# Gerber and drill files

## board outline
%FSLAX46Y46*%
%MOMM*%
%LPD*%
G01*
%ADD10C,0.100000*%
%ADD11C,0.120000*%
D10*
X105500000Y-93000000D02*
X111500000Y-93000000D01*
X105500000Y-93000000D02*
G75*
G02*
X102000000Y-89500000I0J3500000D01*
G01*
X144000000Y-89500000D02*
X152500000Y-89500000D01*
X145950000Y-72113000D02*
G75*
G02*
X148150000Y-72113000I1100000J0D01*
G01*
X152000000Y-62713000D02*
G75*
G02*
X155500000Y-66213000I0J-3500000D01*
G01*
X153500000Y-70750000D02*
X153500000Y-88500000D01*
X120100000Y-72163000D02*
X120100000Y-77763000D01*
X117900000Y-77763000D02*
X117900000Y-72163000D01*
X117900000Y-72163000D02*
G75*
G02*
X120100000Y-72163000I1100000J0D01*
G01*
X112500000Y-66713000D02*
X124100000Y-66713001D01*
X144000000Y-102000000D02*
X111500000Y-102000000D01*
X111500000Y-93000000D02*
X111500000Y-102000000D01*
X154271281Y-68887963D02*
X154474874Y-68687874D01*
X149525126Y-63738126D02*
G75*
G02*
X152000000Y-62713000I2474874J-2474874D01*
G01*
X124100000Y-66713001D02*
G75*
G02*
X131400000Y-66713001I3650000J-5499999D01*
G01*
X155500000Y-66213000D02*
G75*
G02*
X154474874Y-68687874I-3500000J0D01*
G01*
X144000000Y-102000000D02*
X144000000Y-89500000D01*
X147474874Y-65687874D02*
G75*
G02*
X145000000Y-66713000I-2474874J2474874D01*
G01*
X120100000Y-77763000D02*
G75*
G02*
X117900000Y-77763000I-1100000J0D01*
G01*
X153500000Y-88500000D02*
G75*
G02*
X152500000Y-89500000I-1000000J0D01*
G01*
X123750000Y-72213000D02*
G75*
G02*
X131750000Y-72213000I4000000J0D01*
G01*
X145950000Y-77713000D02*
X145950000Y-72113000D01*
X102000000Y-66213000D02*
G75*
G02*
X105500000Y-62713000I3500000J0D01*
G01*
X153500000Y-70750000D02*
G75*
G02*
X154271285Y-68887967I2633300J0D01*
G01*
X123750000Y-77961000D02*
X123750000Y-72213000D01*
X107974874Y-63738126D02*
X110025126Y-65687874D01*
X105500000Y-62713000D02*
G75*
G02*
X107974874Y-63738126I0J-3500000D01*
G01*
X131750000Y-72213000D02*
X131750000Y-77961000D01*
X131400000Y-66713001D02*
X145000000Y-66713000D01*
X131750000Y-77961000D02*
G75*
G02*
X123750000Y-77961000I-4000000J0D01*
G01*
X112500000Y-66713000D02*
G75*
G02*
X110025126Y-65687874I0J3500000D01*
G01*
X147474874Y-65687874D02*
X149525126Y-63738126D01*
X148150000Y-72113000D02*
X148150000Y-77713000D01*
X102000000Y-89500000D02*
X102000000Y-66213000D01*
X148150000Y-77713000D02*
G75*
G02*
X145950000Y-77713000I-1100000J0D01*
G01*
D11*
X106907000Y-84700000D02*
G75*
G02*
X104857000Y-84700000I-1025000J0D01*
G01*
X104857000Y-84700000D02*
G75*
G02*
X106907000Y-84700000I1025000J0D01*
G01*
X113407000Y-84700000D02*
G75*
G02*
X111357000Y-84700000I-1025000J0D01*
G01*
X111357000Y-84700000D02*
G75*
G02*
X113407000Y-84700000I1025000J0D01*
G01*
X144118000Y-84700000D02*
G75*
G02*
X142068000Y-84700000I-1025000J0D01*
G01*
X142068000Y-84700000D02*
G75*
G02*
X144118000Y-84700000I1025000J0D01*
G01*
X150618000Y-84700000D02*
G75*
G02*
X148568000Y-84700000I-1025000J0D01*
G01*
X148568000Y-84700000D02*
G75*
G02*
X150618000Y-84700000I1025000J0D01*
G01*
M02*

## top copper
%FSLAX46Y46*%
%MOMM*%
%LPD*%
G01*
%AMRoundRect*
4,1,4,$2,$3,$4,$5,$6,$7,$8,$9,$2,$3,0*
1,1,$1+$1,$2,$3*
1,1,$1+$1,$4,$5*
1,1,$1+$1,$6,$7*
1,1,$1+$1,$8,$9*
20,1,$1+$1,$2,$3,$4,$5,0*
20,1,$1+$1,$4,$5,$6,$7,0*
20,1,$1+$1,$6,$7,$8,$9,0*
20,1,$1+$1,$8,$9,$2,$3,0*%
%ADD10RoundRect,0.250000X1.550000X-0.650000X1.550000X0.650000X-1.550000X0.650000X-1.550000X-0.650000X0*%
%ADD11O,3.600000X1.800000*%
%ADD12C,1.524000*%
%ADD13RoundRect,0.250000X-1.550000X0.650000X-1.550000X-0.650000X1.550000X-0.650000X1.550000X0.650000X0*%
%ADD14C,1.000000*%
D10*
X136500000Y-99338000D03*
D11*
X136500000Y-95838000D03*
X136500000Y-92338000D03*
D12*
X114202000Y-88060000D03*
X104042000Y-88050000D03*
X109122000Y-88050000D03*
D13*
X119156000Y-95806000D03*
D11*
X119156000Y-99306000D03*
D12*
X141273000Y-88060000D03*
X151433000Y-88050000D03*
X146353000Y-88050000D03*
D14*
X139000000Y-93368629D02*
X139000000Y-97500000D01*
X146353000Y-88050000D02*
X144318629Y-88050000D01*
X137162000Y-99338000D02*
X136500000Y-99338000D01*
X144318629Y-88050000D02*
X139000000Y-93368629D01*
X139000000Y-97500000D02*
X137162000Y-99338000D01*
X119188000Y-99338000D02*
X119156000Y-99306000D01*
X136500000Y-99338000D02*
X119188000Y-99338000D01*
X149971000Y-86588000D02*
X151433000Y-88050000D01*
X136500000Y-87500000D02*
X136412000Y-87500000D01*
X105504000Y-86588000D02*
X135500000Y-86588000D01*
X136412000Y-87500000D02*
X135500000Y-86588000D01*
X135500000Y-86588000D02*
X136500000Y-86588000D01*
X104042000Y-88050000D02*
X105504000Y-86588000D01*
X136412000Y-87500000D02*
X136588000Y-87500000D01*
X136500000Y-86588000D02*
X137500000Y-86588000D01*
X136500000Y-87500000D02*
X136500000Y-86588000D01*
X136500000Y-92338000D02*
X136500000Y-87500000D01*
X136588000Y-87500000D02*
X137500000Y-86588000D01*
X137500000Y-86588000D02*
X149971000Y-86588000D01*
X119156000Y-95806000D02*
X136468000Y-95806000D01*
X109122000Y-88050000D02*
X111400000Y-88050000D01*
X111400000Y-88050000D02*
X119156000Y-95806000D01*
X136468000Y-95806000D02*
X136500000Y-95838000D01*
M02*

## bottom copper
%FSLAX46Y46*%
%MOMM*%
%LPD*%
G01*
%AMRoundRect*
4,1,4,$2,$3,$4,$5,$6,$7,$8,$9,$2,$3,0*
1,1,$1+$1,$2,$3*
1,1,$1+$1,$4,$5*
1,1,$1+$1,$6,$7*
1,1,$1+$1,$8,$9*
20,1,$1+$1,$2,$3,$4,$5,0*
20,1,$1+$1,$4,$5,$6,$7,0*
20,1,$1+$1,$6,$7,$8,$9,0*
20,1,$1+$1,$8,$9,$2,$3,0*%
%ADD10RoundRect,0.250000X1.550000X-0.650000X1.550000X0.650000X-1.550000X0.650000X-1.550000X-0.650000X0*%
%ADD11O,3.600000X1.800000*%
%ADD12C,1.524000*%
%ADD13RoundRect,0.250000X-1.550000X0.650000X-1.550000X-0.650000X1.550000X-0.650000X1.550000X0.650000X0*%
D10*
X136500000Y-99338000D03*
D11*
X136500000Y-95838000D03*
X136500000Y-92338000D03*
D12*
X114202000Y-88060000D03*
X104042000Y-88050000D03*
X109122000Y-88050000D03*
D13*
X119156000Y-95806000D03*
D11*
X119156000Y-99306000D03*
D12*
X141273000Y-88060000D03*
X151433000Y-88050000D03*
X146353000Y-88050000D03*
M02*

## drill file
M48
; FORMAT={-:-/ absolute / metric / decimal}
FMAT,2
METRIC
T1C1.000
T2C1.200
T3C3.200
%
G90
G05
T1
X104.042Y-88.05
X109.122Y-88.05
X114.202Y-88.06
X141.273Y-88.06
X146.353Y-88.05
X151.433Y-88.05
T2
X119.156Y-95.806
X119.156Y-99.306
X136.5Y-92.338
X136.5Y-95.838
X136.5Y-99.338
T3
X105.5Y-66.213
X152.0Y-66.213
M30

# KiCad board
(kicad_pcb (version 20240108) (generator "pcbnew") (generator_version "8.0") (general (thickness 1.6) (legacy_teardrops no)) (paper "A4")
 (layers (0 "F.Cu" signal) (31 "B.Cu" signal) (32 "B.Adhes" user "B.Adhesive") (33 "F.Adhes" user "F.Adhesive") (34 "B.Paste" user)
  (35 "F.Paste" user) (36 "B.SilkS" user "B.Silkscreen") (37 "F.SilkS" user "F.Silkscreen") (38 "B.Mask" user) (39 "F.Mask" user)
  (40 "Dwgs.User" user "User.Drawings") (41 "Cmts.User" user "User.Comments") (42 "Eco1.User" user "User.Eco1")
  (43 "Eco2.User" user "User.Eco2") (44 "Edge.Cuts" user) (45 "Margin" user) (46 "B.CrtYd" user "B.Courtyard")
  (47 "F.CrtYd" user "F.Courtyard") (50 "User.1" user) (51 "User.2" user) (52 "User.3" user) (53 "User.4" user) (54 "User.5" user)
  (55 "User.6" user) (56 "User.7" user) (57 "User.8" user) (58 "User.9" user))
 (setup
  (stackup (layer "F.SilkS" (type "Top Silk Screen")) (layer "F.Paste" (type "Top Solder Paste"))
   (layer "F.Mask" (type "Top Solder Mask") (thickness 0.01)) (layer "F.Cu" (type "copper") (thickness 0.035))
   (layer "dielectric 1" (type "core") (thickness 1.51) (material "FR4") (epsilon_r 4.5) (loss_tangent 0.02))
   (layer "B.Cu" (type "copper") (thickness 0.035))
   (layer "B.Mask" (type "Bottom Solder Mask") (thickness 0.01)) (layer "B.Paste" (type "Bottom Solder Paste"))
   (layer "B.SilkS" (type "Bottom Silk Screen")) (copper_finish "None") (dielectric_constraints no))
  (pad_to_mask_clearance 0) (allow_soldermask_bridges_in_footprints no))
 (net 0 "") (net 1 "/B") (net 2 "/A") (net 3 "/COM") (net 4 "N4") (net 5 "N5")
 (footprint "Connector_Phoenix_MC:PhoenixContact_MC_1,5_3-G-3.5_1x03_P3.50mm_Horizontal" (layer "F.Cu") (at 136.5 99.338 90)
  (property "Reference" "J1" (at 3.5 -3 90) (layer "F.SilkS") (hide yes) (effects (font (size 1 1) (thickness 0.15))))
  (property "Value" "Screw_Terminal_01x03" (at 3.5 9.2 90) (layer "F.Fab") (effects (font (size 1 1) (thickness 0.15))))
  (pad "1" thru_hole roundrect (at 0 0 90) (size 1.8 3.6) (drill 1.2) (layers "*.Cu" "*.Mask") (remove_unused_layers no)
   (roundrect_rratio 0.1388888889) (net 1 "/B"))
  (pad "2" thru_hole oval (at 3.5 0 90) (size 1.8 3.6) (drill 1.2) (layers "*.Cu" "*.Mask") (remove_unused_layers no) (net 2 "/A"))
  (pad "3" thru_hole oval (at 7 0 90) (size 1.8 3.6) (drill 1.2) (layers "*.Cu" "*.Mask") (remove_unused_layers no) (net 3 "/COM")))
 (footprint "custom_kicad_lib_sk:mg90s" (layer "F.Cu") (at 127.674 72.5)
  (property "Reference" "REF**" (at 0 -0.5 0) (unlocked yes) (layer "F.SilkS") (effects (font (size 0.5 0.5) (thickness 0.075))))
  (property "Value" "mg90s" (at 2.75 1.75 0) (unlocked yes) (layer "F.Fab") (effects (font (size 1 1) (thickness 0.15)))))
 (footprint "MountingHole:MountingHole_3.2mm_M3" (layer "F.Cu") (at 152 66.213)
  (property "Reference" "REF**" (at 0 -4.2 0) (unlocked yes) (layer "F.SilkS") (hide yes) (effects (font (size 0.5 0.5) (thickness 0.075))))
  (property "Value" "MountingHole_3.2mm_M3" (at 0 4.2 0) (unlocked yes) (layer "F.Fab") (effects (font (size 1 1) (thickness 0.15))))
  (pad "" np_thru_hole circle (at 0 0) (size 3.2 3.2) (drill 3.2) (layers "*.Cu" "*.Mask")))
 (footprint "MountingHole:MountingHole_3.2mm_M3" (layer "F.Cu") (at 105.5 66.213)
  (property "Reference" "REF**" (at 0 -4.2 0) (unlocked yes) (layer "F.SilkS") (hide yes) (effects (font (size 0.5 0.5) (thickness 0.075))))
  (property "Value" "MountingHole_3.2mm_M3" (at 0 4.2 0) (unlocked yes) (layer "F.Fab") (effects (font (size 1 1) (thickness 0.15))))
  (pad "" np_thru_hole circle (at 0 0) (size 3.2 3.2) (drill 3.2) (layers "F&B.Cu" "*.Mask")))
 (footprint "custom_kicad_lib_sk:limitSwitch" (layer "F.Cu") (at 109.122 87.5)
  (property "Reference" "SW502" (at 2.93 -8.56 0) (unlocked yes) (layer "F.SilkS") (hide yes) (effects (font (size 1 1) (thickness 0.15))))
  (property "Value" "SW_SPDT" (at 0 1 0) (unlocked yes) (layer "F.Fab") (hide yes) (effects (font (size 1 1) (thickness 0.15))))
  (fp_circle (center -3.24 -2.8) (end -2.215 -2.8) (stroke (width 0.12) (type default)) (fill none) (layer "Edge.Cuts"))
  (fp_circle (center 3.26 -2.8) (end 4.285 -2.8) (stroke (width 0.12) (type default)) (fill none) (layer "Edge.Cuts"))
  (pad "1" thru_hole circle (at 5.08 0.56) (size 1.524 1.524) (drill 1) (layers "*.Cu" "*.Mask") (remove_unused_layers no) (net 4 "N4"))
  (pad "2" thru_hole circle (at -5.08 0.55) (size 1.524 1.524) (drill 1) (layers "*.Cu" "*.Mask") (remove_unused_layers no) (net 3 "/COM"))
  (pad "3" thru_hole circle (at 0 0.55) (size 1.524 1.524) (drill 1) (layers "*.Cu" "*.Mask") (remove_unused_layers no) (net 2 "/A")))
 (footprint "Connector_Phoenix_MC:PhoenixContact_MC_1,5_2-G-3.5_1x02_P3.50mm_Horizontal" (layer "F.Cu") (at 119.156 95.806 -90)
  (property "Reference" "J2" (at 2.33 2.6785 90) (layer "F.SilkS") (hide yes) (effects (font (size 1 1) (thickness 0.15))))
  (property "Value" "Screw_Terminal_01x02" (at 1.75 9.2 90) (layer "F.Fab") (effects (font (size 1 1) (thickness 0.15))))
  (pad "1" thru_hole roundrect (at 0 0 270) (size 1.8 3.6) (drill 1.2) (layers "*.Cu" "*.Mask") (remove_unused_layers no)
   (roundrect_rratio 0.1388888889) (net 2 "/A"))
  (pad "2" thru_hole oval (at 3.5 0 270) (size 1.8 3.6) (drill 1.2) (layers "*.Cu" "*.Mask") (remove_unused_layers no) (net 1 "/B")))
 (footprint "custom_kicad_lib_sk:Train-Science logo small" (layer "F.Cu") (at 125.5 87.5)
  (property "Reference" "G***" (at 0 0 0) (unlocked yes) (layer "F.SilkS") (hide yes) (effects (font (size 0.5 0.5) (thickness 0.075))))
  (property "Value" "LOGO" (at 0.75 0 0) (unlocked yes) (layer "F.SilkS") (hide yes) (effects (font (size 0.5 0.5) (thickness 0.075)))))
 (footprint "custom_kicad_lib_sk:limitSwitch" (layer "B.Cu") (at 146.353 87.5 180)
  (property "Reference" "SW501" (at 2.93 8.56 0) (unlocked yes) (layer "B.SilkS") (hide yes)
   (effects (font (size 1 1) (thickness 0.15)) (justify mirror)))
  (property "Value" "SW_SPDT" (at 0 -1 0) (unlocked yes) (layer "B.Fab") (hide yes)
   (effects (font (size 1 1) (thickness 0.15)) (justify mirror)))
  (fp_circle (center 3.26 2.8) (end 4.285 2.8) (stroke (width 0.12) (type default)) (fill none) (layer "Edge.Cuts"))
  (fp_circle (center -3.24 2.8) (end -2.215 2.8) (stroke (width 0.12) (type default)) (fill none) (layer "Edge.Cuts"))
  (pad "1" thru_hole circle (at 5.08 -0.56 180) (size 1.524 1.524) (drill 1) (layers "*.Cu" "*.Mask") (remove_unused_layers no) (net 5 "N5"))
  (pad "2" thru_hole circle (at -5.08 -0.55 180) (size 1.524 1.524) (drill 1) (layers "*.Cu" "*.Mask") (remove_unused_layers no)
   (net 3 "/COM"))
  (pad "3" thru_hole circle (at 0 -0.55 180) (size 1.524 1.524) (drill 1) (layers "*.Cu" "*.Mask") (remove_unused_layers no) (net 1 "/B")))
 (gr_line (start 105.5 93) (end 111.5 93) (stroke (width 0.1) (type default)) (layer "Edge.Cuts"))
 (gr_arc (start 105.5 93) (mid 103.025126 91.974874) (end 102 89.5) (stroke (width 0.1) (type default)) (layer "Edge.Cuts"))
 (gr_line (start 144 89.5) (end 152.5 89.5) (stroke (width 0.1) (type default)) (layer "Edge.Cuts"))
 (gr_arc (start 145.95 72.113) (mid 147.05 71.013) (end 148.15 72.113) (stroke (width 0.1) (type default)) (layer "Edge.Cuts"))
 (gr_arc (start 152 62.713) (mid 154.474874 63.738126) (end 155.5 66.213) (stroke (width 0.1) (type default)) (layer "Edge.Cuts"))
 (gr_line (start 153.5 70.75) (end 153.5 88.5) (stroke (width 0.1) (type default)) (layer "Edge.Cuts"))
 (gr_line (start 120.1 72.163) (end 120.1 77.763) (stroke (width 0.1) (type default)) (layer "Edge.Cuts"))
 (gr_line (start 117.9 77.763) (end 117.9 72.163) (stroke (width 0.1) (type default)) (layer "Edge.Cuts"))
 (gr_arc (start 117.9 72.163) (mid 119 71.063) (end 120.1 72.163) (stroke (width 0.1) (type default)) (layer "Edge.Cuts"))
 (gr_line (start 112.5 66.713) (end 124.1 66.713001) (stroke (width 0.1) (type default)) (layer "Edge.Cuts"))
 (gr_line (start 144 102) (end 111.5 102) (stroke (width 0.1) (type default)) (layer "Edge.Cuts"))
 (gr_line (start 111.5 93) (end 111.5 102) (stroke (width 0.1) (type default)) (layer "Edge.Cuts"))
 (gr_line (start 154.271281 68.887963) (end 154.474874 68.687874) (stroke (width 0.1) (type default)) (layer "Edge.Cuts"))
 (gr_arc (start 149.525126 63.738126) (mid 150.660608 62.979421) (end 152 62.713) (stroke (width 0.1) (type default)) (layer "Edge.Cuts"))
 (gr_arc (start 124.1 66.713001) (mid 127.75 65.612054) (end 131.4 66.713001) (stroke (width 0.1) (type default)) (layer "Edge.Cuts"))
 (gr_arc (start 155.5 66.213) (mid 155.233579 67.552392) (end 154.474874 68.687874) (stroke (width 0.1) (type default)) (layer "Edge.Cuts"))
 (gr_line (start 144 102) (end 144 89.5) (stroke (width 0.1) (type default)) (layer "Edge.Cuts"))
 (gr_arc (start 147.474874 65.687874) (mid 146.339392 66.446579) (end 145 66.713) (stroke (width 0.1) (type default)) (layer "Edge.Cuts"))
 (gr_arc (start 120.1 77.763) (mid 119 78.863) (end 117.9 77.763) (stroke (width 0.1) (type default)) (layer "Edge.Cuts"))
 (gr_arc (start 153.5 88.5) (mid 153.207107 89.207107) (end 152.5 89.5) (stroke (width 0.1) (type default)) (layer "Edge.Cuts"))
 (gr_arc (start 123.75 72.213) (mid 127.75 68.213) (end 131.75 72.213) (stroke (width 0.1) (type default)) (layer "Edge.Cuts"))
 (gr_line (start 145.95 77.713) (end 145.95 72.113) (stroke (width 0.1) (type default)) (layer "Edge.Cuts"))
 (gr_arc (start 102 66.213) (mid 103.025126 63.738126) (end 105.5 62.713) (stroke (width 0.1) (type default)) (layer "Edge.Cuts"))
 (gr_arc (start 153.5 70.75) (mid 153.700449 69.742273) (end 154.271281 68.887963) (stroke (width 0.1) (type default)) (layer "Edge.Cuts"))
 (gr_line (start 123.75 77.961) (end 123.75 72.213) (stroke (width 0.1) (type default)) (layer "Edge.Cuts"))
 (gr_line (start 107.974874 63.738126) (end 110.025126 65.687874) (stroke (width 0.1) (type default)) (layer "Edge.Cuts"))
 (gr_arc (start 105.5 62.713) (mid 106.839392 62.979422) (end 107.974874 63.738126) (stroke (width 0.1) (type default)) (layer "Edge.Cuts"))
 (gr_line (start 131.75 72.213) (end 131.75 77.961) (stroke (width 0.1) (type default)) (layer "Edge.Cuts"))
 (gr_line (start 131.4 66.713001) (end 145 66.713) (stroke (width 0.1) (type default)) (layer "Edge.Cuts"))
 (gr_arc (start 131.75 77.961) (mid 127.75 81.961) (end 123.75 77.961) (stroke (width 0.1) (type default)) (layer "Edge.Cuts"))
 (gr_arc (start 112.5 66.713) (mid 111.160608 66.446578) (end 110.025126 65.687874) (stroke (width 0.1) (type default)) (layer "Edge.Cuts"))
 (gr_line (start 147.474874 65.687874) (end 149.525126 63.738126) (stroke (width 0.1) (type default)) (layer "Edge.Cuts"))
 (gr_line (start 148.15 72.113) (end 148.15 77.713) (stroke (width 0.1) (type default)) (layer "Edge.Cuts"))
 (gr_line (start 102 89.5) (end 102 66.213) (stroke (width 0.1) (type default)) (layer "Edge.Cuts"))
 (gr_arc (start 148.15 77.713) (mid 147.05 78.813) (end 145.95 77.713) (stroke (width 0.1) (type default)) (layer "Edge.Cuts"))
 (segment (start 139 93.368629) (end 139 97.5) (width 1) (layer "F.Cu") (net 1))
 (segment (start 146.353 88.05) (end 144.318629 88.05) (width 1) (layer "F.Cu") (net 1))
 (segment (start 137.162 99.338) (end 136.5 99.338) (width 1) (layer "F.Cu") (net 1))
 (segment (start 144.318629 88.05) (end 139 93.368629) (width 1) (layer "F.Cu") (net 1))
 (segment (start 139 97.5) (end 137.162 99.338) (width 1) (layer "F.Cu") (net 1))
 (segment (start 119.188 99.338) (end 119.156 99.306) (width 1) (layer "F.Cu") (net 1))
 (segment (start 136.5 99.338) (end 119.188 99.338) (width 1) (layer "F.Cu") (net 1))
 (segment (start 149.971 86.588) (end 151.433 88.05) (width 1) (layer "F.Cu") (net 3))
 (segment (start 136.5 87.5) (end 136.412 87.5) (width 1) (layer "F.Cu") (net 3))
 (segment (start 105.504 86.588) (end 135.5 86.588) (width 1) (layer "F.Cu") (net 3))
 (segment (start 136.412 87.5) (end 135.5 86.588) (width 1) (layer "F.Cu") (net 3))
 (segment (start 135.5 86.588) (end 136.5 86.588) (width 1) (layer "F.Cu") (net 3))
 (segment (start 104.042 88.05) (end 105.504 86.588) (width 1) (layer "F.Cu") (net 3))
 (segment (start 136.412 87.5) (end 136.588 87.5) (width 1) (layer "F.Cu") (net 3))
 (segment (start 136.5 86.588) (end 137.5 86.588) (width 1) (layer "F.Cu") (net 3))
 (segment (start 136.5 87.5) (end 136.5 86.588) (width 1) (layer "F.Cu") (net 3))
 (segment (start 136.5 92.338) (end 136.5 87.5) (width 1) (layer "F.Cu") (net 3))
 (segment (start 136.588 87.5) (end 137.5 86.588) (width 1) (layer "F.Cu") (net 3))
 (segment (start 137.5 86.588) (end 149.971 86.588) (width 1) (layer "F.Cu") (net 3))
 (segment (start 119.156 95.806) (end 136.468 95.806) (width 1) (layer "F.Cu") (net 2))
 (segment (start 109.122 88.05) (end 111.4 88.05) (width 1) (layer "F.Cu") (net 2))
 (segment (start 111.4 88.05) (end 119.156 95.806) (width 1) (layer "F.Cu") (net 2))
 (segment (start 136.468 95.806) (end 136.5 95.838) (width 1) (layer "F.Cu") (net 2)))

